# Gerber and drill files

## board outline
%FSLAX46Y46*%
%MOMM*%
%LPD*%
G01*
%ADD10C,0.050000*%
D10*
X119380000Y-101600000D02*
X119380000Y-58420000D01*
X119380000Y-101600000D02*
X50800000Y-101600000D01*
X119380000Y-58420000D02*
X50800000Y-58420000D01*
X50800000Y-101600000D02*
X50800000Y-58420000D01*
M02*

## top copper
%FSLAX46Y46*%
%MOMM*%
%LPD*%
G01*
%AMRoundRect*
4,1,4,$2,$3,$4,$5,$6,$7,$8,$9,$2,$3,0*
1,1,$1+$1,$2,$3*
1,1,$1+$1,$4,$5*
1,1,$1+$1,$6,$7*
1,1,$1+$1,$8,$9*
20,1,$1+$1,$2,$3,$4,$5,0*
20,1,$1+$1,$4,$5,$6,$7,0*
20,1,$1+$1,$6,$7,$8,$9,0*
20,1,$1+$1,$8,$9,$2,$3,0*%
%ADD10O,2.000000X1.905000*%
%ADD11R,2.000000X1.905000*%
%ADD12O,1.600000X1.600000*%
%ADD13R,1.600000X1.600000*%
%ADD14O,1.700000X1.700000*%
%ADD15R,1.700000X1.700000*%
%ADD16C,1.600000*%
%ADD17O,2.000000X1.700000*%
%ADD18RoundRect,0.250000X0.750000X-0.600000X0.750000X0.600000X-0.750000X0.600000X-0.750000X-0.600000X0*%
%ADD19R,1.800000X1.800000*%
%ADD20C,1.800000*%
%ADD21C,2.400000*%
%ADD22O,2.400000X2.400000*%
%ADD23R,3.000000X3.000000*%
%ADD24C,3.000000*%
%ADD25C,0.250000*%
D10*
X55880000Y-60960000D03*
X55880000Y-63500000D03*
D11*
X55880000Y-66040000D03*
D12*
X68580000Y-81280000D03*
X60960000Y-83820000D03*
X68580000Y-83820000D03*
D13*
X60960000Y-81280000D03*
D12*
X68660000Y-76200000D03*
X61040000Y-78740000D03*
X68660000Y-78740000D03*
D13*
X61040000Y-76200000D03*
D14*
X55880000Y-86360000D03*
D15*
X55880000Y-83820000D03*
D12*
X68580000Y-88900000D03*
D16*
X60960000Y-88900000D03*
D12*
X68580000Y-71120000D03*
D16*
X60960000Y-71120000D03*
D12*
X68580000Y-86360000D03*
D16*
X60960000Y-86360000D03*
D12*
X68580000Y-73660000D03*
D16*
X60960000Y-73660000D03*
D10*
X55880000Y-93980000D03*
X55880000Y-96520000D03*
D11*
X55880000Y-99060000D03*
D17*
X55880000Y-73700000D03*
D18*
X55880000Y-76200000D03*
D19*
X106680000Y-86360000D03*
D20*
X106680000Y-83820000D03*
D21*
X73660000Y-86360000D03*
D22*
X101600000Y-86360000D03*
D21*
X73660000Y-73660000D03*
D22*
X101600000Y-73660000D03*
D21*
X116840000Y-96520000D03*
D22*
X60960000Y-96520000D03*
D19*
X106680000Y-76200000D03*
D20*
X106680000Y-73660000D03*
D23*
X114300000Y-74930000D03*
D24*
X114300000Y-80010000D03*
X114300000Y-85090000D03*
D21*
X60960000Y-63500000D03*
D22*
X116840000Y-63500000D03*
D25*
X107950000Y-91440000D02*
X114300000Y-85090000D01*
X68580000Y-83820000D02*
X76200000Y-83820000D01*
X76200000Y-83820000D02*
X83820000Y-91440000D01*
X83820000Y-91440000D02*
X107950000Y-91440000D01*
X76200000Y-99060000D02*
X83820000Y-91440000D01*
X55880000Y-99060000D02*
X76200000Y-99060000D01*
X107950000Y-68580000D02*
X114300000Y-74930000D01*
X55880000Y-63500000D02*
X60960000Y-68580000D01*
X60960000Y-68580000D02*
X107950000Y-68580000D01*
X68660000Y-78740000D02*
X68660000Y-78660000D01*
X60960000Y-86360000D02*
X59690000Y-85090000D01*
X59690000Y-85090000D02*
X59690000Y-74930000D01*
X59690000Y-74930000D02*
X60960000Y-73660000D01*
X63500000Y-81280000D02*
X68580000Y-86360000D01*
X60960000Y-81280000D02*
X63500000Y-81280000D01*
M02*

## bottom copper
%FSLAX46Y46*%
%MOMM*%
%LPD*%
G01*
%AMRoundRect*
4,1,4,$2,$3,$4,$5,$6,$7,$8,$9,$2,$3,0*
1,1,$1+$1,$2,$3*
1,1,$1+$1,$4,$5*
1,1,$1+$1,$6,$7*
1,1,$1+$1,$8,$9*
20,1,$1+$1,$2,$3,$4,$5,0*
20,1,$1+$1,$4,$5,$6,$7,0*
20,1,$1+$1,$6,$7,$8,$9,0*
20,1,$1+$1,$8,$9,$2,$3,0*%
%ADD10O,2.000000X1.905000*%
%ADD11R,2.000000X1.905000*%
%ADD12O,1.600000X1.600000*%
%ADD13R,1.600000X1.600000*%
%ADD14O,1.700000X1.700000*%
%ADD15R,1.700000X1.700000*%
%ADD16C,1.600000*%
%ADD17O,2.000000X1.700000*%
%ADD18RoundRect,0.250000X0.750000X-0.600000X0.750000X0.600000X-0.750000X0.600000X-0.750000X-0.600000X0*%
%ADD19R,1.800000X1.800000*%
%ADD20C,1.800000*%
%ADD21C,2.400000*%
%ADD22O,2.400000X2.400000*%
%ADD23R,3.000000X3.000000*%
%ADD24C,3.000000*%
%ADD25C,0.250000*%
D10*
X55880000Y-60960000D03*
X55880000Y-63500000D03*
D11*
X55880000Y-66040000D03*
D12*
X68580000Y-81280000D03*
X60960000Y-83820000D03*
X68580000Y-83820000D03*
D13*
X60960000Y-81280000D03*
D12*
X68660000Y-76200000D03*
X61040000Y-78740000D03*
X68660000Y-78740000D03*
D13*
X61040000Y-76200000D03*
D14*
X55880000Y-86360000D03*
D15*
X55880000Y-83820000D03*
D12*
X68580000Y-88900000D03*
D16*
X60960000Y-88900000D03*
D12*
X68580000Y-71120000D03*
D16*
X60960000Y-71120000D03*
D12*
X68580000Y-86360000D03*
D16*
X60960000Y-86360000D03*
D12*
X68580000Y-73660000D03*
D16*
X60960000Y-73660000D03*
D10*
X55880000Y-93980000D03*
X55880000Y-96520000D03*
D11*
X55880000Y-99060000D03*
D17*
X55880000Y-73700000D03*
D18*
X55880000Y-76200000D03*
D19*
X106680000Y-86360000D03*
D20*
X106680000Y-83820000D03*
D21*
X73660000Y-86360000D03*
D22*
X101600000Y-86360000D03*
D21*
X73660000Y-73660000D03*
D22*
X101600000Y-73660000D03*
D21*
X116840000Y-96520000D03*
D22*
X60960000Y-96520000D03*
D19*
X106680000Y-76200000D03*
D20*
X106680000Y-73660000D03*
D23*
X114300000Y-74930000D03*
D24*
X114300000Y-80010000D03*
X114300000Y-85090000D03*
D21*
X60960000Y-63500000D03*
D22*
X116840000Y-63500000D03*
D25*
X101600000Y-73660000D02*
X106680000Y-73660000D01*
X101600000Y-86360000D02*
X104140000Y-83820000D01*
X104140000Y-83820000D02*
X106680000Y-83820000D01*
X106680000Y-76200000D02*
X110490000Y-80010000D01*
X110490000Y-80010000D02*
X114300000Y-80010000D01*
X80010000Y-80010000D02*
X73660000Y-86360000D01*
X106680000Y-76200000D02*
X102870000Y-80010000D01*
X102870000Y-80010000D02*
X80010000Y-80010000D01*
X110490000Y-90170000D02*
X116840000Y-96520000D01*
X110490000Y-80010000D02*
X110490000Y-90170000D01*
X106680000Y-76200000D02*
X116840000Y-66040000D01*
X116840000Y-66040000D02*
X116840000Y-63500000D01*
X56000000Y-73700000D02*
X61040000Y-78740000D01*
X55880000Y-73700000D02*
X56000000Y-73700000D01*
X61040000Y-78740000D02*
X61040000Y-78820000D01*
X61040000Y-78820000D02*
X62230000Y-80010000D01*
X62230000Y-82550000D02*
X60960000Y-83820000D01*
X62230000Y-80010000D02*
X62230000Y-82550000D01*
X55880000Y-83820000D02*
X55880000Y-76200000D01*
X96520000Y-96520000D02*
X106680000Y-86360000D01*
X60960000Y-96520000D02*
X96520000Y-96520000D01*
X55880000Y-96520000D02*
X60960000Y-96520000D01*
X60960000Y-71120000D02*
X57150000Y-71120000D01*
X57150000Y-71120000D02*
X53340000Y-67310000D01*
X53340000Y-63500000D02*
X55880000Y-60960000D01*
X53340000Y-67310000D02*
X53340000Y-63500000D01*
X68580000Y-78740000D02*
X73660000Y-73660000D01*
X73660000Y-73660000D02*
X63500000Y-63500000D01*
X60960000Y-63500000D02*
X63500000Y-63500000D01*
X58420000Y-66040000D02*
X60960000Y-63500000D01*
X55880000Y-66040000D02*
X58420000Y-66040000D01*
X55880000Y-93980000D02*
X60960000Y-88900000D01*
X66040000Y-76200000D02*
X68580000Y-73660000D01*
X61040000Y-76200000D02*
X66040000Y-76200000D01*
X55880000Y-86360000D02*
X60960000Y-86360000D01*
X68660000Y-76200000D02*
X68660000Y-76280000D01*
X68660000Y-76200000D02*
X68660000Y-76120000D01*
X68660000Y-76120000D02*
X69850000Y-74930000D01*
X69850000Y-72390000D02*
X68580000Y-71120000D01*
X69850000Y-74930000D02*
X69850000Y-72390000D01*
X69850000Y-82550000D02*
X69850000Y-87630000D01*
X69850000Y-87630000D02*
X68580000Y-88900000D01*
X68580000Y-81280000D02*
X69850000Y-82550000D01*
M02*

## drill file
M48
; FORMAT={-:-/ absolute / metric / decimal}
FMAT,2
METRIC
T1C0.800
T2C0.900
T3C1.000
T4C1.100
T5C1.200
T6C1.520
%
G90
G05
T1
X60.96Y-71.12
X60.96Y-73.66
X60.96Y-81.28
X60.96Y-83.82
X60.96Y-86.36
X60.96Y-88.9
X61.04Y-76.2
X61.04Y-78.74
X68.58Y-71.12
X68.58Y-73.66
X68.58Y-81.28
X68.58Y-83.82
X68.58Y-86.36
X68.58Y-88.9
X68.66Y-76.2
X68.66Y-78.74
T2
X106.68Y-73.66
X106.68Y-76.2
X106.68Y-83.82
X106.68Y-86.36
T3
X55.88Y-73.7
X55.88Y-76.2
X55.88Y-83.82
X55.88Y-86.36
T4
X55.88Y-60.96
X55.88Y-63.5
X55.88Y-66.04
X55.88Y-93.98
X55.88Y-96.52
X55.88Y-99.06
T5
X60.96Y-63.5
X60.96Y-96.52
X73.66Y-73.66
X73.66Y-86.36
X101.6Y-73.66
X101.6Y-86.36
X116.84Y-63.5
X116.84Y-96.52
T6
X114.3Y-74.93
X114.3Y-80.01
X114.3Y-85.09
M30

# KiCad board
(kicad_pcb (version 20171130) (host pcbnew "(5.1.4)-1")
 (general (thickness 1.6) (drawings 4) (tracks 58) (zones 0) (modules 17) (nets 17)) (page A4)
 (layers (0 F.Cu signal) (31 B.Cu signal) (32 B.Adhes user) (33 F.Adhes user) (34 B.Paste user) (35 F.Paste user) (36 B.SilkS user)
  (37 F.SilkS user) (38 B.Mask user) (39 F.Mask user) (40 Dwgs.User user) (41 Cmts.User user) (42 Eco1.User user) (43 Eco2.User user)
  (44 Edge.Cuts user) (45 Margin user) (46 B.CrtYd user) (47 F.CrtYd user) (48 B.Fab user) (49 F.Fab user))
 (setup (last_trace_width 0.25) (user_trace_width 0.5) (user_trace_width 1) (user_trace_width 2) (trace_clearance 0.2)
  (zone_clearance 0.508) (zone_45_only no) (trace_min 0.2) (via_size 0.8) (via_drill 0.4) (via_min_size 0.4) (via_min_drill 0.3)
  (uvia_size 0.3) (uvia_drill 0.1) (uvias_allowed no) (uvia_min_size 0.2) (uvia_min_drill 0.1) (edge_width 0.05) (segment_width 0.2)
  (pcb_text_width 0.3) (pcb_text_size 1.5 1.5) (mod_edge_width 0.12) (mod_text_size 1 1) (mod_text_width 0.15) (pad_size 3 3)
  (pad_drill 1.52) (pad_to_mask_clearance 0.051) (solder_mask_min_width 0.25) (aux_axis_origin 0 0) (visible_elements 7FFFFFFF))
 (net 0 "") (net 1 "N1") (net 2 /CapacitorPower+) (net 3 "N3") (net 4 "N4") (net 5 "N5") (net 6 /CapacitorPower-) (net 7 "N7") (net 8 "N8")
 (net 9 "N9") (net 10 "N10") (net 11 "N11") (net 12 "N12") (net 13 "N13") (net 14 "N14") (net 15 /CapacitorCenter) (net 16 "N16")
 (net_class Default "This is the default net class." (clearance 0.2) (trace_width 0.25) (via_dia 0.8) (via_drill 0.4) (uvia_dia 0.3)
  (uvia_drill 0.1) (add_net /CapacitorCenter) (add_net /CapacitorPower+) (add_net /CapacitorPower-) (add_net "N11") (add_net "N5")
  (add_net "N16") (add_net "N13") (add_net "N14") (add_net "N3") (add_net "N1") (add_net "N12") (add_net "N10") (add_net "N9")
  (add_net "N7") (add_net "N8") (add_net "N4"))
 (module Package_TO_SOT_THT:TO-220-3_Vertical (layer F.Cu) (at 55.88 66.04 90)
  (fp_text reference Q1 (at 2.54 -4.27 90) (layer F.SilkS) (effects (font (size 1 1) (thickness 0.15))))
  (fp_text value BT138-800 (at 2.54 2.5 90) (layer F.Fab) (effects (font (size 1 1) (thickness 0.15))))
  (pad 3 thru_hole oval (at 5.08 0 90) (size 1.905 2) (drill 1.1) (layers *.Cu *.Mask) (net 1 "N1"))
  (pad 2 thru_hole oval (at 2.54 0 90) (size 1.905 2) (drill 1.1) (layers *.Cu *.Mask) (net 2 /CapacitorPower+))
  (pad 1 thru_hole rect (at 0 0 90) (size 1.905 2) (drill 1.1) (layers *.Cu *.Mask) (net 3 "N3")))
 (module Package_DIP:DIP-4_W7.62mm (layer F.Cu) (at 60.96 81.28)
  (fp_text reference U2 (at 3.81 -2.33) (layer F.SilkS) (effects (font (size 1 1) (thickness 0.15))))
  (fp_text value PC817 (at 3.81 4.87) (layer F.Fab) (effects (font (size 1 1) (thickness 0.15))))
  (pad 4 thru_hole oval (at 7.62 0) (size 1.6 1.6) (drill 0.8) (layers *.Cu *.Mask) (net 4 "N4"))
  (pad 2 thru_hole oval (at 0 2.54) (size 1.6 1.6) (drill 0.8) (layers *.Cu *.Mask) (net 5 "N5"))
  (pad 3 thru_hole oval (at 7.62 2.54) (size 1.6 1.6) (drill 0.8) (layers *.Cu *.Mask) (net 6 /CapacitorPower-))
  (pad 1 thru_hole rect (at 0 0) (size 1.6 1.6) (drill 0.8) (layers *.Cu *.Mask) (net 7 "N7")))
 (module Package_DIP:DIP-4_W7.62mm (layer F.Cu) (at 61.04 76.2)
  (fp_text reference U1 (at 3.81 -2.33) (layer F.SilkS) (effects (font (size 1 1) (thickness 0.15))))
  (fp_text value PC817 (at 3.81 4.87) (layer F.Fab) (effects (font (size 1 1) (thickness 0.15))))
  (pad 4 thru_hole oval (at 7.62 0) (size 1.6 1.6) (drill 0.8) (layers *.Cu *.Mask) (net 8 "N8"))
  (pad 2 thru_hole oval (at 0 2.54) (size 1.6 1.6) (drill 0.8) (layers *.Cu *.Mask) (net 5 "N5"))
  (pad 3 thru_hole oval (at 7.62 2.54) (size 1.6 1.6) (drill 0.8) (layers *.Cu *.Mask) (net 3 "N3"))
  (pad 1 thru_hole rect (at 0 0) (size 1.6 1.6) (drill 0.8) (layers *.Cu *.Mask) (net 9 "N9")))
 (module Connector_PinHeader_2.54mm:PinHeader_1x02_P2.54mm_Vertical (layer F.Cu) (at 55.88 83.82)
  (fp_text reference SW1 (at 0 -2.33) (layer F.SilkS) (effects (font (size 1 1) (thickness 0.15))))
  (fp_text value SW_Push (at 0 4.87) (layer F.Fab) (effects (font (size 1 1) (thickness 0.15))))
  (pad 2 thru_hole oval (at 0 2.54) (size 1.7 1.7) (drill 1) (layers *.Cu *.Mask) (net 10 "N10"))
  (pad 1 thru_hole rect (at 0 0) (size 1.7 1.7) (drill 1) (layers *.Cu *.Mask) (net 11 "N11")))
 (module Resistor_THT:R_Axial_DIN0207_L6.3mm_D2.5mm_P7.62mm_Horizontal (layer F.Cu) (at 60.96 88.9)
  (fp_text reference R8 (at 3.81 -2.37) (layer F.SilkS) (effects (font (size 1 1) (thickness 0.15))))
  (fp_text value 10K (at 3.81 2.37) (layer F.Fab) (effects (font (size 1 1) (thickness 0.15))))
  (pad 2 thru_hole oval (at 7.62 0) (size 1.6 1.6) (drill 0.8) (layers *.Cu *.Mask) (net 4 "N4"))
  (pad 1 thru_hole circle (at 0 0) (size 1.6 1.6) (drill 0.8) (layers *.Cu *.Mask) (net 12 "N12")))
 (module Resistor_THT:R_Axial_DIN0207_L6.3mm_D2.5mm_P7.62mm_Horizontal (layer F.Cu) (at 60.96 71.12)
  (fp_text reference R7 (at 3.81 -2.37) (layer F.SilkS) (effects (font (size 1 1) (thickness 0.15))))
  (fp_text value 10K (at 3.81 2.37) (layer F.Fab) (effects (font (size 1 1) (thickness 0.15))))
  (pad 2 thru_hole oval (at 7.62 0) (size 1.6 1.6) (drill 0.8) (layers *.Cu *.Mask) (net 8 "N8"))
  (pad 1 thru_hole circle (at 0 0) (size 1.6 1.6) (drill 0.8) (layers *.Cu *.Mask) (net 1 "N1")))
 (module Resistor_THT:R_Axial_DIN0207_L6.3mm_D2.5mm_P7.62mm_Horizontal (layer F.Cu) (at 60.96 86.36)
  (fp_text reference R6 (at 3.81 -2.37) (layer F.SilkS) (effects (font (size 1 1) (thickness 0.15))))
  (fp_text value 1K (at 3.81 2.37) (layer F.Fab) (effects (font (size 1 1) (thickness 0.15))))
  (pad 2 thru_hole oval (at 7.62 0) (size 1.6 1.6) (drill 0.8) (layers *.Cu *.Mask) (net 7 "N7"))
  (pad 1 thru_hole circle (at 0 0) (size 1.6 1.6) (drill 0.8) (layers *.Cu *.Mask) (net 10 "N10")))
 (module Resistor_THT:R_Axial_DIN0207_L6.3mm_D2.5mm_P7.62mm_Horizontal (layer F.Cu) (at 60.96 73.66)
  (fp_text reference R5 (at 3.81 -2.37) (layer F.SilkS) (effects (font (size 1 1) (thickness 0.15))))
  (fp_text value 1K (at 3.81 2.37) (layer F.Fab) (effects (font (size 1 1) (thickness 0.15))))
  (pad 2 thru_hole oval (at 7.62 0) (size 1.6 1.6) (drill 0.8) (layers *.Cu *.Mask) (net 9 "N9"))
  (pad 1 thru_hole circle (at 0 0) (size 1.6 1.6) (drill 0.8) (layers *.Cu *.Mask) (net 10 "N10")))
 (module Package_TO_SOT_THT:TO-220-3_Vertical (layer F.Cu) (at 55.88 99.06 90)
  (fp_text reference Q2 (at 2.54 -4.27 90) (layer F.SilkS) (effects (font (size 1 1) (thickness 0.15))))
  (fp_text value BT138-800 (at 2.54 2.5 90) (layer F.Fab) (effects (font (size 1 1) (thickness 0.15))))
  (pad 3 thru_hole oval (at 5.08 0 90) (size 1.905 2) (drill 1.1) (layers *.Cu *.Mask) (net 12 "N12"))
  (pad 2 thru_hole oval (at 2.54 0 90) (size 1.905 2) (drill 1.1) (layers *.Cu *.Mask) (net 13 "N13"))
  (pad 1 thru_hole rect (at 0 0 90) (size 1.905 2) (drill 1.1) (layers *.Cu *.Mask) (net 6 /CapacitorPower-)))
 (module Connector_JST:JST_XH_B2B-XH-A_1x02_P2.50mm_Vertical (layer F.Cu) (at 55.88 76.2 90)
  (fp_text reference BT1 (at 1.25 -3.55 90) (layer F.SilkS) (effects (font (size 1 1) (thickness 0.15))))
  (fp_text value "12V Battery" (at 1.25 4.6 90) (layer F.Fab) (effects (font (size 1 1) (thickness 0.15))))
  (pad 2 thru_hole oval (at 2.5 0 90) (size 1.7 2) (drill 1) (layers *.Cu *.Mask) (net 5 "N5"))
  (pad 1 thru_hole roundrect (at 0 0 90) (size 1.7 2) (drill 1) (layers *.Cu *.Mask) (roundrect_rratio 0.147059) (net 11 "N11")))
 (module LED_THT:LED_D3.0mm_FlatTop (layer F.Cu) (at 106.68 86.36 90)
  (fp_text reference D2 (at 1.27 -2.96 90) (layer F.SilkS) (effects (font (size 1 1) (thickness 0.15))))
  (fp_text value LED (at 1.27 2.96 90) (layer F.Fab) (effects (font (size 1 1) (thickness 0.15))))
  (pad 1 thru_hole rect (at 0 0 90) (size 1.8 1.8) (drill 0.9) (layers *.Cu *.Mask) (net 13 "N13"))
  (pad 2 thru_hole circle (at 2.54 0 90) (size 1.8 1.8) (drill 0.9) (layers *.Cu *.Mask) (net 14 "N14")))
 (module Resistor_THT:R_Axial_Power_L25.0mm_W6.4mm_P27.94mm (layer F.Cu) (at 73.66 86.36)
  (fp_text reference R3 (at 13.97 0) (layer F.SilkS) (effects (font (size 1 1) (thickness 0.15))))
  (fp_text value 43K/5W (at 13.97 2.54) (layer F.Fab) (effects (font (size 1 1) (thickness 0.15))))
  (pad 1 thru_hole circle (at 0 0) (size 2.4 2.4) (drill 1.2) (layers *.Cu *.Mask) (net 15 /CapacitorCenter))
  (pad 2 thru_hole oval (at 27.94 0) (size 2.4 2.4) (drill 1.2) (layers *.Cu *.Mask) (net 14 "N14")))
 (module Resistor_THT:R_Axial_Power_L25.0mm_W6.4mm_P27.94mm (layer F.Cu) (at 73.66 73.66)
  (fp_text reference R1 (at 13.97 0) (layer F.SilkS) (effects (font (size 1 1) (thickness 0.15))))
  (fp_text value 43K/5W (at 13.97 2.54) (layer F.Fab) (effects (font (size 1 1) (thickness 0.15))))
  (pad 1 thru_hole circle (at 0 0) (size 2.4 2.4) (drill 1.2) (layers *.Cu *.Mask) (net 3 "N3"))
  (pad 2 thru_hole oval (at 27.94 0) (size 2.4 2.4) (drill 1.2) (layers *.Cu *.Mask) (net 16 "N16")))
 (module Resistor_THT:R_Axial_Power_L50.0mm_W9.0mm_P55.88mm (layer F.Cu) (at 116.84 96.52 180)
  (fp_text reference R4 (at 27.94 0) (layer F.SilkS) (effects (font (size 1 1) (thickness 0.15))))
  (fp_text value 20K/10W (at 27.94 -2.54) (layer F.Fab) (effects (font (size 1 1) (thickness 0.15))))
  (pad 1 thru_hole circle (at 0 0 180) (size 2.4 2.4) (drill 1.2) (layers *.Cu *.Mask) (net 15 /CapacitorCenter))
  (pad 2 thru_hole oval (at 55.88 0 180) (size 2.4 2.4) (drill 1.2) (layers *.Cu *.Mask) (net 13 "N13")))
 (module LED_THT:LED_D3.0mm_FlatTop (layer F.Cu) (at 106.68 76.2 90)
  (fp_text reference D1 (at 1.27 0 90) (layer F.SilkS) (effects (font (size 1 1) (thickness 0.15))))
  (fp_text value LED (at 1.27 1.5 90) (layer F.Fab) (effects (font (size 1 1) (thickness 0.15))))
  (pad 1 thru_hole rect (at 0 0 90) (size 1.8 1.8) (drill 0.9) (layers *.Cu *.Mask) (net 15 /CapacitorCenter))
  (pad 2 thru_hole circle (at 2.54 0 90) (size 1.8 1.8) (drill 0.9) (layers *.Cu *.Mask) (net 16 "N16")))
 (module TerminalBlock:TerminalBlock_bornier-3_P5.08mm (layer F.Cu) (at 114.3 74.93 270)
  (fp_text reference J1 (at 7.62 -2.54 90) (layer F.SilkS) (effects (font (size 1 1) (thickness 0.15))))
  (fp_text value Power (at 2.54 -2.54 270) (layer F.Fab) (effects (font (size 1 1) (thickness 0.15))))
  (pad 1 thru_hole rect (at 0 0 270) (size 3 3) (drill 1.52) (layers *.Cu *.Mask) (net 2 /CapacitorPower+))
  (pad 2 thru_hole circle (at 5.08 0 270) (size 3 3) (drill 1.52) (layers *.Cu *.Mask) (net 15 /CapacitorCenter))
  (pad 3 thru_hole circle (at 10.16 0 270) (size 3 3) (drill 1.52) (layers *.Cu *.Mask) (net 6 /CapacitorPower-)))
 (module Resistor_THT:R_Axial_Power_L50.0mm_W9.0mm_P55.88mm (layer F.Cu) (at 60.96 63.5)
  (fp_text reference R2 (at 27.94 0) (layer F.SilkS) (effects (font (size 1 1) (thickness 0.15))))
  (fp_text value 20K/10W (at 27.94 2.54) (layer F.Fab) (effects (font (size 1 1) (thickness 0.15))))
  (pad 1 thru_hole circle (at 0 0) (size 2.4 2.4) (drill 1.2) (layers *.Cu *.Mask) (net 3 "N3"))
  (pad 2 thru_hole oval (at 55.88 0) (size 2.4 2.4) (drill 1.2) (layers *.Cu *.Mask) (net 15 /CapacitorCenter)))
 (gr_line (start 119.38 101.6) (end 119.38 58.42) (layer Edge.Cuts) (width 0.05))
 (gr_line (start 119.38 101.6) (end 50.8 101.6) (layer Edge.Cuts) (width 0.05))
 (gr_line (start 119.38 58.42) (end 50.8 58.42) (layer Edge.Cuts) (width 0.05))
 (gr_line (start 50.8 101.6) (end 50.8 58.42) (layer Edge.Cuts) (width 0.05))
 (segment (start 101.6 73.66) (end 106.68 73.66) (width 0.25) (layer B.Cu) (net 16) (status 30))
 (segment (start 101.6 86.36) (end 104.14 83.82) (width 0.25) (layer B.Cu) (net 14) (status 10))
 (segment (start 104.14 83.82) (end 106.68 83.82) (width 0.25) (layer B.Cu) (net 14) (status 20))
 (segment (start 106.68 76.2) (end 110.49 80.01) (width 0.25) (layer B.Cu) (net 15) (status 10))
 (segment (start 110.49 80.01) (end 114.3 80.01) (width 0.25) (layer B.Cu) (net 15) (status 20))
 (segment (start 80.01 80.01) (end 73.66 86.36) (width 0.25) (layer B.Cu) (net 15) (status 20))
 (segment (start 106.68 76.2) (end 102.87 80.01) (width 0.25) (layer B.Cu) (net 15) (status 10))
 (segment (start 102.87 80.01) (end 80.01 80.01) (width 0.25) (layer B.Cu) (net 15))
 (segment (start 110.49 90.17) (end 116.84 96.52) (width 0.25) (layer B.Cu) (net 15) (status 20))
 (segment (start 110.49 80.01) (end 110.49 90.17) (width 0.25) (layer B.Cu) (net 15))
 (segment (start 106.68 76.2) (end 116.84 66.04) (width 0.25) (layer B.Cu) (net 15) (status 10))
 (segment (start 116.84 66.04) (end 116.84 63.5) (width 0.25) (layer B.Cu) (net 15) (status 20))
 (segment (start 107.95 91.44) (end 114.3 85.09) (width 0.25) (layer F.Cu) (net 6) (status 20))
 (segment (start 68.58 83.82) (end 76.2 83.82) (width 0.25) (layer F.Cu) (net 6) (status 10))
 (segment (start 76.2 83.82) (end 83.82 91.44) (width 0.25) (layer F.Cu) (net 6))
 (segment (start 83.82 91.44) (end 107.95 91.44) (width 0.25) (layer F.Cu) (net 6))
 (segment (start 76.2 99.06) (end 83.82 91.44) (width 0.25) (layer F.Cu) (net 6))
 (segment (start 55.88 99.06) (end 76.2 99.06) (width 0.25) (layer F.Cu) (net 6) (status 10))
 (segment (start 107.95 68.58) (end 114.3 74.93) (width 0.25) (layer F.Cu) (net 2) (status 20))
 (segment (start 55.88 63.5) (end 60.96 68.58) (width 0.25) (layer F.Cu) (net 2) (status 10))
 (segment (start 60.96 68.58) (end 107.95 68.58) (width 0.25) (layer F.Cu) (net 2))
 (segment (start 56 73.7) (end 61.04 78.74) (width 0.25) (layer B.Cu) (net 5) (status 30))
 (segment (start 55.88 73.7) (end 56 73.7) (width 0.25) (layer B.Cu) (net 5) (status 30))
 (segment (start 61.04 78.74) (end 61.04 78.82) (width 0.25) (layer B.Cu) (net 5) (status 30))
 (segment (start 61.04 78.82) (end 62.23 80.01) (width 0.25) (layer B.Cu) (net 5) (status 10))
 (segment (start 62.23 82.55) (end 60.96 83.82) (width 0.25) (layer B.Cu) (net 5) (status 20))
 (segment (start 62.23 80.01) (end 62.23 82.55) (width 0.25) (layer B.Cu) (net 5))
 (segment (start 55.88 83.82) (end 55.88 76.2) (width 0.25) (layer B.Cu) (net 11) (status 30))
 (segment (start 96.52 96.52) (end 106.68 86.36) (width 0.25) (layer B.Cu) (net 13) (status 20))
 (segment (start 60.96 96.52) (end 96.52 96.52) (width 0.25) (layer B.Cu) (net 13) (status 10))
 (segment (start 55.88 96.52) (end 60.96 96.52) (width 0.25) (layer B.Cu) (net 13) (status 30))
 (segment (start 60.96 71.12) (end 57.15 71.12) (width 0.25) (layer B.Cu) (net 1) (status 10))
 (segment (start 57.15 71.12) (end 53.34 67.31) (width 0.25) (layer B.Cu) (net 1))
 (segment (start 53.34 63.5) (end 55.88 60.96) (width 0.25) (layer B.Cu) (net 1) (status 20))
 (segment (start 53.34 67.31) (end 53.34 63.5) (width 0.25) (layer B.Cu) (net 1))
 (segment (start 68.66 78.74) (end 68.66 78.66) (width 0.25) (layer F.Cu) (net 3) (status 30))
 (segment (start 68.58 78.74) (end 73.66 73.66) (width 0.25) (layer B.Cu) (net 3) (status 30))
 (segment (start 73.66 73.66) (end 63.5 63.5) (width 0.25) (layer B.Cu) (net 3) (status 10))
 (segment (start 60.96 63.5) (end 63.5 63.5) (width 0.25) (layer B.Cu) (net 3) (status 10))
 (segment (start 58.42 66.04) (end 60.96 63.5) (width 0.25) (layer B.Cu) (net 3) (status 20))
 (segment (start 55.88 66.04) (end 58.42 66.04) (width 0.25) (layer B.Cu) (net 3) (status 10))
 (segment (start 55.88 93.98) (end 60.96 88.9) (width 0.25) (layer B.Cu) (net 12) (status 30))
 (segment (start 66.04 76.2) (end 68.58 73.66) (width 0.25) (layer B.Cu) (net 9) (status 20))
 (segment (start 61.04 76.2) (end 66.04 76.2) (width 0.25) (layer B.Cu) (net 9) (status 10))
 (segment (start 55.88 86.36) (end 60.96 86.36) (width 0.25) (layer B.Cu) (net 10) (status 30))
 (segment (start 60.96 86.36) (end 59.69 85.09) (width 0.25) (layer F.Cu) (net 10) (status 10))
 (segment (start 59.69 85.09) (end 59.69 74.93) (width 0.25) (layer F.Cu) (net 10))
 (segment (start 59.69 74.93) (end 60.96 73.66) (width 0.25) (layer F.Cu) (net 10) (status 20))
 (segment (start 63.5 81.28) (end 68.58 86.36) (width 0.25) (layer F.Cu) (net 7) (status 20))
 (segment (start 60.96 81.28) (end 63.5 81.28) (width 0.25) (layer F.Cu) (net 7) (status 10))
 (segment (start 68.66 76.2) (end 68.66 76.28) (width 0.25) (layer B.Cu) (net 8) (status 30))
 (segment (start 68.66 76.2) (end 68.66 76.12) (width 0.25) (layer B.Cu) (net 8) (status 30))
 (segment (start 68.66 76.12) (end 69.85 74.93) (width 0.25) (layer B.Cu) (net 8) (status 10))
 (segment (start 69.85 72.39) (end 68.58 71.12) (width 0.25) (layer B.Cu) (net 8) (status 20))
 (segment (start 69.85 74.93) (end 69.85 72.39) (width 0.25) (layer B.Cu) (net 8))
 (segment (start 69.85 82.55) (end 69.85 87.63) (width 0.25) (layer B.Cu) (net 4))
 (segment (start 69.85 87.63) (end 68.58 88.9) (width 0.25) (layer B.Cu) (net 4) (status 20))
 (segment (start 68.58 81.28) (end 69.85 82.55) (width 0.25) (layer B.Cu) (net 4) (status 10)))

